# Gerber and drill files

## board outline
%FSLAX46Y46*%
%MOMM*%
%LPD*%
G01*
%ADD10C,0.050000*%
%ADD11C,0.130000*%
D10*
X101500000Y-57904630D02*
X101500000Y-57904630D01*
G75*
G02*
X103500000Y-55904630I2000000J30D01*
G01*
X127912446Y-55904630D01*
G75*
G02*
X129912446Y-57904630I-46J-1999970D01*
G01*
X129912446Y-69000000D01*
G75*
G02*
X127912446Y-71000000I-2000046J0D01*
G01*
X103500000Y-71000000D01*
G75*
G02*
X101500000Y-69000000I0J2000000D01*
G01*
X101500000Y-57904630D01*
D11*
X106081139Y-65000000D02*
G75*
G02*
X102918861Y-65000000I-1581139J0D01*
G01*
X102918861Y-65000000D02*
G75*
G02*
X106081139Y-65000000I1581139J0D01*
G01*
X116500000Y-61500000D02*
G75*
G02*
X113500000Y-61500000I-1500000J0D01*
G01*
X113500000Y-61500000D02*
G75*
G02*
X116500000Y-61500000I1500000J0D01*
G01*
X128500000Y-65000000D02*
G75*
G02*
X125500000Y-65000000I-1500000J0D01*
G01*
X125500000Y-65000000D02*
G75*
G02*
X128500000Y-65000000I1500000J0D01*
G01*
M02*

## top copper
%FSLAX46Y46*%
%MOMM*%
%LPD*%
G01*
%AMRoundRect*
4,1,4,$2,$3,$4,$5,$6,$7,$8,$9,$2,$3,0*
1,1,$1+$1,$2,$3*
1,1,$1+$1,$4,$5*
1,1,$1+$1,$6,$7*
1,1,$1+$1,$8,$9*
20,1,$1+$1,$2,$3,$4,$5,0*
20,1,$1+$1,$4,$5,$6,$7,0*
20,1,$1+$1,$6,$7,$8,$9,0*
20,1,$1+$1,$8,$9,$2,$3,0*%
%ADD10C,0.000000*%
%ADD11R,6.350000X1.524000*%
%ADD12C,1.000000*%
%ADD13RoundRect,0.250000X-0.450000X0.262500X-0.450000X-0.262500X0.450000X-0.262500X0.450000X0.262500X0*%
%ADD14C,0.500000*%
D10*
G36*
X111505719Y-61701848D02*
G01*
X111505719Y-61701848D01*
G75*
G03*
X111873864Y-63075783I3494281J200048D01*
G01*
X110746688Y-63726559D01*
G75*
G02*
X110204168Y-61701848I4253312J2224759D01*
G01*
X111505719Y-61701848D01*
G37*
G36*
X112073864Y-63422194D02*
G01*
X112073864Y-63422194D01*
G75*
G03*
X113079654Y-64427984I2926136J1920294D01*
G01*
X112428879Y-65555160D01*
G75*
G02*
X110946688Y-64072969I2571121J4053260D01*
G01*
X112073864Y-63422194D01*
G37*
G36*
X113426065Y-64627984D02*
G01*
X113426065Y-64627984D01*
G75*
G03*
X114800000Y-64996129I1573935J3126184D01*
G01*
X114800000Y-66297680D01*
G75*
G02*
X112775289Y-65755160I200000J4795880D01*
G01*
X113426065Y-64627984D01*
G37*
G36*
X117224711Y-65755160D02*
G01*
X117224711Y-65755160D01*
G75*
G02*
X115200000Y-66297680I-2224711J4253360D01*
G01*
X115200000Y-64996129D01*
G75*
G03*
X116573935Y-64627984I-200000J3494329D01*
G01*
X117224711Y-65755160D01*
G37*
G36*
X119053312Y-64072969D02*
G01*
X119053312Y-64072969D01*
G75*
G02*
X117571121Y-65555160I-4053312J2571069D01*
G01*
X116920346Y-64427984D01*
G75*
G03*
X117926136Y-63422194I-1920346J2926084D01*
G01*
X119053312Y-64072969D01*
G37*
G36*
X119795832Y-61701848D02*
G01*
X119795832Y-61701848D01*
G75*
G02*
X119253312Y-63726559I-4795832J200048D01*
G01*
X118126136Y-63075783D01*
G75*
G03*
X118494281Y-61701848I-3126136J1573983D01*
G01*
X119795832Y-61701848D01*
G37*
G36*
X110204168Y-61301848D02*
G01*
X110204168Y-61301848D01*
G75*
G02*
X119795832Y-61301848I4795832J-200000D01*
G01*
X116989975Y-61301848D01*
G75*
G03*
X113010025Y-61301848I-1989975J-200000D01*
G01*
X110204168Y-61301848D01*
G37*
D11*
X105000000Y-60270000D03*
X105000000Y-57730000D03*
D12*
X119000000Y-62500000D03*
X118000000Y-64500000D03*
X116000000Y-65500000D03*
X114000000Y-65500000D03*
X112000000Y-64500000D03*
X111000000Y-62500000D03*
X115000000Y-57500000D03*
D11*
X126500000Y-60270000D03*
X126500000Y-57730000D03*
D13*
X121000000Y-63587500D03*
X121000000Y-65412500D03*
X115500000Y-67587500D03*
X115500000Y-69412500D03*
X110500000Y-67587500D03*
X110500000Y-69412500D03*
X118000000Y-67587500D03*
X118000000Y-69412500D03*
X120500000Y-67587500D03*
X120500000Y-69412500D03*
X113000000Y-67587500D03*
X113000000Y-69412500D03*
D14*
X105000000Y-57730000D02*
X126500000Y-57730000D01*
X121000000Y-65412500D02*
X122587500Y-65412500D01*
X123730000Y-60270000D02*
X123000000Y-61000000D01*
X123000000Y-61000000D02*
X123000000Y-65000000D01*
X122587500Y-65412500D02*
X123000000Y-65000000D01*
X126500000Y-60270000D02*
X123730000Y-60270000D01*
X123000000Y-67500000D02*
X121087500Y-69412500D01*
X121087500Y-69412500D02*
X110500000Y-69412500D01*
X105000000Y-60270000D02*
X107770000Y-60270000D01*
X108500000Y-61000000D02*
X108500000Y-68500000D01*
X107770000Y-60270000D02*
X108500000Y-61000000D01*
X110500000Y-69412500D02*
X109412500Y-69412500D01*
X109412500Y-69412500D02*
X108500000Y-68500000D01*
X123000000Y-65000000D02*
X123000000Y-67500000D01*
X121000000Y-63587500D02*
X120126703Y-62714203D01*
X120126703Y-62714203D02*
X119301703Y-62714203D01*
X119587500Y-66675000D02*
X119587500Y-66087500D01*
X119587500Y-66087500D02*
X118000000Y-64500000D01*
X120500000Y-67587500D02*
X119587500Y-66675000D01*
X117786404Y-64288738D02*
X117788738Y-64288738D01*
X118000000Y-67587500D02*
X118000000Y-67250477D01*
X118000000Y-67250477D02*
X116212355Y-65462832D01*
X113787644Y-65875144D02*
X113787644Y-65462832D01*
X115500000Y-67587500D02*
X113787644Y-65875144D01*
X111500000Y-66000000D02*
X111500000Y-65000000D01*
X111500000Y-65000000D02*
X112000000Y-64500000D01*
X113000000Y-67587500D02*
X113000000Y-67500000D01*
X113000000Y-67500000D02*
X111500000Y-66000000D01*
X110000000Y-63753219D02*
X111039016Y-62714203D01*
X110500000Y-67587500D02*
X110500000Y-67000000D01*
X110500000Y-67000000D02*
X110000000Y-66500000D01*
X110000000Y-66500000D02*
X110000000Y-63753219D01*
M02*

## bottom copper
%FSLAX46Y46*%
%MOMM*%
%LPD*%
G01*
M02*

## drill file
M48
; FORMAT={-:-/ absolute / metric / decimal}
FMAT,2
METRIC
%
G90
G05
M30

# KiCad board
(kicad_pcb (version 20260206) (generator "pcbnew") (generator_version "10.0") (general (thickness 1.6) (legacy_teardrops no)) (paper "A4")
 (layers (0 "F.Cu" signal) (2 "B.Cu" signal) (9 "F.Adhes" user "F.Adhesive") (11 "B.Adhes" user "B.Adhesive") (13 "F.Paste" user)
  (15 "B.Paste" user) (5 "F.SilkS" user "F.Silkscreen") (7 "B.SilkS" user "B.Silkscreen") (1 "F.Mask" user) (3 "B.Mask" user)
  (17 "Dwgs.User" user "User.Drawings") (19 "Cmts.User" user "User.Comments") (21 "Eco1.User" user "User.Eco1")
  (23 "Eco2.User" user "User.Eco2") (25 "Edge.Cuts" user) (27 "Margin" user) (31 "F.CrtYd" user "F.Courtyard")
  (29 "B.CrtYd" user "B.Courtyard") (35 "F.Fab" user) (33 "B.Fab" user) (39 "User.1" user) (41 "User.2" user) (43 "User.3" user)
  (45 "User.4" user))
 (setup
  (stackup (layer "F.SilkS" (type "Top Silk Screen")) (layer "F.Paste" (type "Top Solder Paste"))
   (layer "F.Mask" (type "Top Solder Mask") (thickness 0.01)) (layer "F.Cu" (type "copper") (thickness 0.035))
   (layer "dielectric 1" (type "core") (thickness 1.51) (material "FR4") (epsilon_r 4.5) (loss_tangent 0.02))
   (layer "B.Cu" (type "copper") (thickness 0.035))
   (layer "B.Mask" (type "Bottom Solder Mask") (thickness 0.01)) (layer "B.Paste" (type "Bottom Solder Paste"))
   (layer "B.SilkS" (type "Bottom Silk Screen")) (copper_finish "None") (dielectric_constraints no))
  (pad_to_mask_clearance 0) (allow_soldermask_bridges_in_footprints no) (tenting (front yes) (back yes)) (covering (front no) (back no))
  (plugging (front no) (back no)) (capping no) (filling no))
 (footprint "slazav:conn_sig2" (layer "F.Cu") (at 105 59 180)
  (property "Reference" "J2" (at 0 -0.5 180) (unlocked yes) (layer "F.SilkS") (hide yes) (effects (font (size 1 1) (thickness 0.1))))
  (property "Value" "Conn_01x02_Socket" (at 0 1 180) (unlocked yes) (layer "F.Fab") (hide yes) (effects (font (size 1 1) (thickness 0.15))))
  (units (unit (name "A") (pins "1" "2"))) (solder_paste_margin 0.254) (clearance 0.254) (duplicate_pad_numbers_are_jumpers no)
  (pad "1" smd rect (at 0 -1.27 180) (size 6.35 1.524) (layers "F.Cu" "F.Mask" "F.Paste") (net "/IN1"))
  (pad "2" smd rect (at 0 1.27 180) (size 6.35 1.524) (layers "F.Cu" "F.Mask" "F.Paste") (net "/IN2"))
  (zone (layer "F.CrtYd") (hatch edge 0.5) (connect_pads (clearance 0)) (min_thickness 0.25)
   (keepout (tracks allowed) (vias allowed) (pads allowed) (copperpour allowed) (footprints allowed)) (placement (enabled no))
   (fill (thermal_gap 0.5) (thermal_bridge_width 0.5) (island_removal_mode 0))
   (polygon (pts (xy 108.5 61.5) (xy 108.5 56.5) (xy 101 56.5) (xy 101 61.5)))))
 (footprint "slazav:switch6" (layer "F.Cu") (at 115 61.5 180)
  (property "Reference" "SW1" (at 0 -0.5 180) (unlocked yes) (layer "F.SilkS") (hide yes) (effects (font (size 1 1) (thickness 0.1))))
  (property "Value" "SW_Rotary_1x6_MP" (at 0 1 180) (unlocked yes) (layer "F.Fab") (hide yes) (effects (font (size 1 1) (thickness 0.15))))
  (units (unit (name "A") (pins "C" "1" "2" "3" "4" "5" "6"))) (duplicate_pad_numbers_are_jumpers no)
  (pad "1" smd circle (at -4 -1 180) (size 1 1) (layers "F.Cu" "F.Mask" "F.Paste") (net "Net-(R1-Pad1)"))
  (pad "2" smd circle (at -3 -3 180) (size 1 1) (layers "F.Cu" "F.Mask" "F.Paste") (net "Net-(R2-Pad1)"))
  (pad "3" smd circle (at -1 -4 180) (size 1 1) (layers "F.Cu" "F.Mask" "F.Paste") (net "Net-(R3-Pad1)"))
  (pad "4" smd circle (at 1 -4 180) (size 1 1) (layers "F.Cu" "F.Mask" "F.Paste") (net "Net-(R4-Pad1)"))
  (pad "5" smd circle (at 3 -3 180) (size 1 1) (layers "F.Cu" "F.Mask" "F.Paste") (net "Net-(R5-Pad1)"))
  (pad "6" smd circle (at 4 -1 180) (size 1 1) (layers "F.Cu" "F.Mask" "F.Paste") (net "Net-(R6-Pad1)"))
  (pad "C" smd circle (at 0 4 180) (size 1 1) (layers "F.Cu" "F.Mask" "F.Paste") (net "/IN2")))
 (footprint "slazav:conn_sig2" (layer "F.Cu") (at 126.5 59 180)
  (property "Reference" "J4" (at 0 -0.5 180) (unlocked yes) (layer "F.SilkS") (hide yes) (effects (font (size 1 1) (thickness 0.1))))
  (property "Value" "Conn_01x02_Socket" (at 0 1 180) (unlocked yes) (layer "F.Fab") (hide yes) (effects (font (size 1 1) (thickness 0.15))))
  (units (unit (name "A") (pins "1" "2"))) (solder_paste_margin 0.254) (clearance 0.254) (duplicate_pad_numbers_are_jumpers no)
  (pad "1" smd rect (at 0 -1.27 180) (size 6.35 1.524) (layers "F.Cu" "F.Mask" "F.Paste") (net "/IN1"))
  (pad "2" smd rect (at 0 1.27 180) (size 6.35 1.524) (layers "F.Cu" "F.Mask" "F.Paste") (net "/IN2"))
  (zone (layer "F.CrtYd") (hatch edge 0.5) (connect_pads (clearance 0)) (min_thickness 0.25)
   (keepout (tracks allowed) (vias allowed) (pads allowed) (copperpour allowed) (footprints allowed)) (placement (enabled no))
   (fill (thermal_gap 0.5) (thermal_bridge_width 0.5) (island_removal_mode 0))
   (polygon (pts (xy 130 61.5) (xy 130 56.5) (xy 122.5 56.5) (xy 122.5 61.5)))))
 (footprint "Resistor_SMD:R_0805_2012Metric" (layer "F.Cu") (at 121 64.5 -90)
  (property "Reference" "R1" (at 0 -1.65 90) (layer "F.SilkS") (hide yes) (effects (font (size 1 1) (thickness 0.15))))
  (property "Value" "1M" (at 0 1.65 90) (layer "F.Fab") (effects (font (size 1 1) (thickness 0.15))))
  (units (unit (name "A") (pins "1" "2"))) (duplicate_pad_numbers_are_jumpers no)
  (pad "1" smd roundrect (at -0.9125 0 270) (size 1.025 1.4) (layers "F.Cu" "F.Mask" "F.Paste") (roundrect_rratio 0.243902)
   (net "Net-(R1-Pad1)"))
  (pad "2" smd roundrect (at 0.9125 0 270) (size 1.025 1.4) (layers "F.Cu" "F.Mask" "F.Paste") (roundrect_rratio 0.243902) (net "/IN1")))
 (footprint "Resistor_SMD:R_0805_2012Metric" (layer "F.Cu") (at 115.5 68.5 -90)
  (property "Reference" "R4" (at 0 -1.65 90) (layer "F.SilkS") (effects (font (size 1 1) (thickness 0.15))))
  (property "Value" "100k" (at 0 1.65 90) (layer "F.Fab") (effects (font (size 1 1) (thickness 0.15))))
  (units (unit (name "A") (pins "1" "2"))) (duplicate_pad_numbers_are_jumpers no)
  (pad "1" smd roundrect (at -0.9125 0 270) (size 1.025 1.4) (layers "F.Cu" "F.Mask" "F.Paste") (roundrect_rratio 0.243902)
   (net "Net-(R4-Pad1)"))
  (pad "2" smd roundrect (at 0.9125 0 270) (size 1.025 1.4) (layers "F.Cu" "F.Mask" "F.Paste") (roundrect_rratio 0.243902) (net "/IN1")))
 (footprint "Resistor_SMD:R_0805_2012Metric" (layer "F.Cu") (at 110.5 68.5 -90)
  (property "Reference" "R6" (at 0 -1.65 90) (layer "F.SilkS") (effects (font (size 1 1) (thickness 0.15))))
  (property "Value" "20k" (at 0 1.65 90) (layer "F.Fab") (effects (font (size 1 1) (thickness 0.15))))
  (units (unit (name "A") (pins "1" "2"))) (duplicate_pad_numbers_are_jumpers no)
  (pad "1" smd roundrect (at -0.9125 0 270) (size 1.025 1.4) (layers "F.Cu" "F.Mask" "F.Paste") (roundrect_rratio 0.243902)
   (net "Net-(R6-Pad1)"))
  (pad "2" smd roundrect (at 0.9125 0 270) (size 1.025 1.4) (layers "F.Cu" "F.Mask" "F.Paste") (roundrect_rratio 0.243902) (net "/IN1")))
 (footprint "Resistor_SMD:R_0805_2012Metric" (layer "F.Cu") (at 118 68.5 -90)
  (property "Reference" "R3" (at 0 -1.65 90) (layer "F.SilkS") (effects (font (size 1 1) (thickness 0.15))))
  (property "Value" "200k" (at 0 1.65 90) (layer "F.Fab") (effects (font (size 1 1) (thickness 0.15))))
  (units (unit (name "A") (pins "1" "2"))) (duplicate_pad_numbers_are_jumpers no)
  (pad "1" smd roundrect (at -0.9125 0 270) (size 1.025 1.4) (layers "F.Cu" "F.Mask" "F.Paste") (roundrect_rratio 0.243902)
   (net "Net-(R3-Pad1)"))
  (pad "2" smd roundrect (at 0.9125 0 270) (size 1.025 1.4) (layers "F.Cu" "F.Mask" "F.Paste") (roundrect_rratio 0.243902) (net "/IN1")))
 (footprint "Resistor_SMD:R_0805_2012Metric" (layer "F.Cu") (at 120.5 68.5 -90)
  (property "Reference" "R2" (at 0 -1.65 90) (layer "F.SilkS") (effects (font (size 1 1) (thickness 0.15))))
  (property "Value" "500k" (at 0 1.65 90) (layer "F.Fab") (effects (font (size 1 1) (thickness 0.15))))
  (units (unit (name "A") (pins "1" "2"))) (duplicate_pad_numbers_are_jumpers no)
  (pad "1" smd roundrect (at -0.9125 0 270) (size 1.025 1.4) (layers "F.Cu" "F.Mask" "F.Paste") (roundrect_rratio 0.243902)
   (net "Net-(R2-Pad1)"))
  (pad "2" smd roundrect (at 0.9125 0 270) (size 1.025 1.4) (layers "F.Cu" "F.Mask" "F.Paste") (roundrect_rratio 0.243902) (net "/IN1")))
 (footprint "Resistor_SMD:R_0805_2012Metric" (layer "F.Cu") (at 113 68.5 -90)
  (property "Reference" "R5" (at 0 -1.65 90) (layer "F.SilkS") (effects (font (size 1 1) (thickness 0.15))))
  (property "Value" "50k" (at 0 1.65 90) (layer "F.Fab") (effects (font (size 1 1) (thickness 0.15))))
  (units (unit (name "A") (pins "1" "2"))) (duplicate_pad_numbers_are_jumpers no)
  (pad "1" smd roundrect (at -0.9125 0 270) (size 1.025 1.4) (layers "F.Cu" "F.Mask" "F.Paste") (roundrect_rratio 0.243902)
   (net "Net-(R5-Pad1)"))
  (pad "2" smd roundrect (at 0.9125 0 270) (size 1.025 1.4) (layers "F.Cu" "F.Mask" "F.Paste") (roundrect_rratio 0.243902) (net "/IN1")))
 (gr_poly
  (pts
   (arc (start 111.505719 61.701848) (mid 111.61926 62.407714) (end 111.873864 63.075783))
   (arc (start 110.746688 63.726559) (mid 110.363556 62.744179) (end 110.204168 61.701848)))
  (stroke (width 0) (type solid)) (fill yes) (layer "F.Cu") (net "Net-(R6-Pad1)"))
 (gr_poly
  (pts
   (arc (start 112.073864 63.422194) (mid 112.525126 63.976722) (end 113.079654 64.427984))
   (arc (start 112.428879 65.55516) (mid 111.605887 64.895961) (end 110.946688 64.072969)))
  (stroke (width 0) (type solid)) (fill yes) (layer "F.Cu") (net "Net-(R5-Pad1)"))
 (gr_poly
  (pts
   (arc (start 113.426065 64.627984) (mid 114.094134 64.882588) (end 114.8 64.996129))
   (arc (start 114.8 66.29768) (mid 113.757668 66.138292) (end 112.775289 65.75516)))
  (stroke (width 0) (type solid)) (fill yes) (layer "F.Cu") (net "Net-(R4-Pad1)"))
 (gr_poly
  (pts
   (arc (start 115.2 64.996129) (mid 115.905866 64.882588) (end 116.573935 64.627984))
   (arc (start 117.224711 65.75516) (mid 116.242331 66.138292) (end 115.2 66.29768)))
  (stroke (width 0) (type solid)) (fill yes) (layer "F.Cu") (net "Net-(R3-Pad1)"))
 (gr_poly
  (pts
   (arc (start 116.920346 64.427984) (mid 117.474874 63.976722) (end 117.926136 63.422194))
   (arc (start 119.053312 64.072969) (mid 118.394113 64.895961) (end 117.571121 65.55516)))
  (stroke (width 0) (type solid)) (fill yes) (layer "F.Cu") (net "Net-(R2-Pad1)"))
 (gr_poly
  (pts
   (arc (start 119.795832 61.701848) (mid 119.636444 62.74418) (end 119.253312 63.726559))
   (arc (start 118.126136 63.075783) (mid 118.38074 62.407714) (end 118.494281 61.701848)))
  (stroke (width 0) (type solid)) (fill yes) (layer "F.Cu") (net "Net-(R1-Pad1)"))
 (gr_poly
  (pts
   (arc (start 119.795832 61.301848) (mid 115 56.701848) (end 110.204168 61.301848))
   (arc (start 113.010025 61.301848) (mid 115 59.501848) (end 116.989975 61.301848)))
  (stroke (width 0) (type solid)) (fill yes) (layer "F.Cu") (net "/IN2"))
 (gr_rect (start 101.5 55.90463) (end 129.912446 71) (radius 2) (stroke (width 0.05) (type solid)) (fill no) (layer "Edge.Cuts"))
 (gr_circle (center 104.5 65) (end 106 65.5) (stroke (width 0.13) (type solid)) (fill no) (layer "Edge.Cuts"))
 (gr_circle (center 115 61.5) (end 116.5 61.5) (stroke (width 0.13) (type solid)) (fill no) (layer "Edge.Cuts"))
 (gr_circle (center 127 65) (end 128.5 65) (stroke (width 0.13) (type solid)) (fill no) (layer "Edge.Cuts"))
 (segment (start 105 57.73) (end 126.5 57.73) (width 0.5) (layer "F.Cu") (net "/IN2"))
 (segment (start 121 65.4125) (end 122.5875 65.4125) (width 0.5) (layer "F.Cu") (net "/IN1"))
 (segment (start 123.73 60.27) (end 123 61) (width 0.5) (layer "F.Cu") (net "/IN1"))
 (segment (start 123 61) (end 123 65) (width 0.5) (layer "F.Cu") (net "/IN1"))
 (segment (start 122.5875 65.4125) (end 123 65) (width 0.5) (layer "F.Cu") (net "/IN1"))
 (segment (start 126.5 60.27) (end 123.73 60.27) (width 0.5) (layer "F.Cu") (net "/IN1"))
 (segment (start 123 67.5) (end 121.0875 69.4125) (width 0.5) (layer "F.Cu") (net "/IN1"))
 (segment (start 121.0875 69.4125) (end 110.5 69.4125) (width 0.5) (layer "F.Cu") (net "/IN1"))
 (segment (start 105 60.27) (end 107.77 60.27) (width 0.5) (layer "F.Cu") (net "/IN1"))
 (segment (start 108.5 61) (end 108.5 68.5) (width 0.5) (layer "F.Cu") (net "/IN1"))
 (segment (start 107.77 60.27) (end 108.5 61) (width 0.5) (layer "F.Cu") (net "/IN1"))
 (segment (start 110.5 69.4125) (end 109.4125 69.4125) (width 0.5) (layer "F.Cu") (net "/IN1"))
 (segment (start 109.4125 69.4125) (end 108.5 68.5) (width 0.5) (layer "F.Cu") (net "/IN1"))
 (segment (start 123 65) (end 123 67.5) (width 0.5) (layer "F.Cu") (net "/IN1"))
 (segment (start 121 63.5875) (end 120.126703 62.714203) (width 0.5) (layer "F.Cu") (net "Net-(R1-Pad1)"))
 (segment (start 120.126703 62.714203) (end 119.301703 62.714203) (width 0.5) (layer "F.Cu") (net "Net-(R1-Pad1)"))
 (segment (start 119.5875 66.675) (end 119.5875 66.0875) (width 0.5) (layer "F.Cu") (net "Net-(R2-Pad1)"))
 (segment (start 119.5875 66.0875) (end 118 64.5) (width 0.5) (layer "F.Cu") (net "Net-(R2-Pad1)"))
 (segment (start 120.5 67.5875) (end 119.5875 66.675) (width 0.5) (layer "F.Cu") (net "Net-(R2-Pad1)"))
 (segment (start 117.786404 64.288738) (end 117.788738 64.288738) (width 0.5) (layer "F.Cu") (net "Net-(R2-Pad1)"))
 (segment (start 118 67.5875) (end 118 67.250477) (width 0.5) (layer "F.Cu") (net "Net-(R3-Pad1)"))
 (segment (start 118 67.250477) (end 116.212355 65.462832) (width 0.5) (layer "F.Cu") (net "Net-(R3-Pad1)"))
 (segment (start 113.787644 65.875144) (end 113.787644 65.462832) (width 0.5) (layer "F.Cu") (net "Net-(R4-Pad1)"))
 (segment (start 115.5 67.5875) (end 113.787644 65.875144) (width 0.5) (layer "F.Cu") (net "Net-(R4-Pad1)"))
 (segment (start 111.5 66) (end 111.5 65) (width 0.5) (layer "F.Cu") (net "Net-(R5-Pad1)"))
 (segment (start 111.5 65) (end 112 64.5) (width 0.5) (layer "F.Cu") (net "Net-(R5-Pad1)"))
 (segment (start 113 67.5875) (end 113 67.5) (width 0.5) (layer "F.Cu") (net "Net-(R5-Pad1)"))
 (segment (start 113 67.5) (end 111.5 66) (width 0.5) (layer "F.Cu") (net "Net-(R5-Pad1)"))
 (segment (start 110 63.753219) (end 111.039016 62.714203) (width 0.5) (layer "F.Cu") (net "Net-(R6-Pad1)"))
 (segment (start 110.5 67.5875) (end 110.5 67) (width 0.5) (layer "F.Cu") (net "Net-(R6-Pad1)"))
 (segment (start 110.5 67) (end 110 66.5) (width 0.5) (layer "F.Cu") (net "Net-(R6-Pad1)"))
 (segment (start 110 66.5) (end 110 63.753219) (width 0.5) (layer "F.Cu") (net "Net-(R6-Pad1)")))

